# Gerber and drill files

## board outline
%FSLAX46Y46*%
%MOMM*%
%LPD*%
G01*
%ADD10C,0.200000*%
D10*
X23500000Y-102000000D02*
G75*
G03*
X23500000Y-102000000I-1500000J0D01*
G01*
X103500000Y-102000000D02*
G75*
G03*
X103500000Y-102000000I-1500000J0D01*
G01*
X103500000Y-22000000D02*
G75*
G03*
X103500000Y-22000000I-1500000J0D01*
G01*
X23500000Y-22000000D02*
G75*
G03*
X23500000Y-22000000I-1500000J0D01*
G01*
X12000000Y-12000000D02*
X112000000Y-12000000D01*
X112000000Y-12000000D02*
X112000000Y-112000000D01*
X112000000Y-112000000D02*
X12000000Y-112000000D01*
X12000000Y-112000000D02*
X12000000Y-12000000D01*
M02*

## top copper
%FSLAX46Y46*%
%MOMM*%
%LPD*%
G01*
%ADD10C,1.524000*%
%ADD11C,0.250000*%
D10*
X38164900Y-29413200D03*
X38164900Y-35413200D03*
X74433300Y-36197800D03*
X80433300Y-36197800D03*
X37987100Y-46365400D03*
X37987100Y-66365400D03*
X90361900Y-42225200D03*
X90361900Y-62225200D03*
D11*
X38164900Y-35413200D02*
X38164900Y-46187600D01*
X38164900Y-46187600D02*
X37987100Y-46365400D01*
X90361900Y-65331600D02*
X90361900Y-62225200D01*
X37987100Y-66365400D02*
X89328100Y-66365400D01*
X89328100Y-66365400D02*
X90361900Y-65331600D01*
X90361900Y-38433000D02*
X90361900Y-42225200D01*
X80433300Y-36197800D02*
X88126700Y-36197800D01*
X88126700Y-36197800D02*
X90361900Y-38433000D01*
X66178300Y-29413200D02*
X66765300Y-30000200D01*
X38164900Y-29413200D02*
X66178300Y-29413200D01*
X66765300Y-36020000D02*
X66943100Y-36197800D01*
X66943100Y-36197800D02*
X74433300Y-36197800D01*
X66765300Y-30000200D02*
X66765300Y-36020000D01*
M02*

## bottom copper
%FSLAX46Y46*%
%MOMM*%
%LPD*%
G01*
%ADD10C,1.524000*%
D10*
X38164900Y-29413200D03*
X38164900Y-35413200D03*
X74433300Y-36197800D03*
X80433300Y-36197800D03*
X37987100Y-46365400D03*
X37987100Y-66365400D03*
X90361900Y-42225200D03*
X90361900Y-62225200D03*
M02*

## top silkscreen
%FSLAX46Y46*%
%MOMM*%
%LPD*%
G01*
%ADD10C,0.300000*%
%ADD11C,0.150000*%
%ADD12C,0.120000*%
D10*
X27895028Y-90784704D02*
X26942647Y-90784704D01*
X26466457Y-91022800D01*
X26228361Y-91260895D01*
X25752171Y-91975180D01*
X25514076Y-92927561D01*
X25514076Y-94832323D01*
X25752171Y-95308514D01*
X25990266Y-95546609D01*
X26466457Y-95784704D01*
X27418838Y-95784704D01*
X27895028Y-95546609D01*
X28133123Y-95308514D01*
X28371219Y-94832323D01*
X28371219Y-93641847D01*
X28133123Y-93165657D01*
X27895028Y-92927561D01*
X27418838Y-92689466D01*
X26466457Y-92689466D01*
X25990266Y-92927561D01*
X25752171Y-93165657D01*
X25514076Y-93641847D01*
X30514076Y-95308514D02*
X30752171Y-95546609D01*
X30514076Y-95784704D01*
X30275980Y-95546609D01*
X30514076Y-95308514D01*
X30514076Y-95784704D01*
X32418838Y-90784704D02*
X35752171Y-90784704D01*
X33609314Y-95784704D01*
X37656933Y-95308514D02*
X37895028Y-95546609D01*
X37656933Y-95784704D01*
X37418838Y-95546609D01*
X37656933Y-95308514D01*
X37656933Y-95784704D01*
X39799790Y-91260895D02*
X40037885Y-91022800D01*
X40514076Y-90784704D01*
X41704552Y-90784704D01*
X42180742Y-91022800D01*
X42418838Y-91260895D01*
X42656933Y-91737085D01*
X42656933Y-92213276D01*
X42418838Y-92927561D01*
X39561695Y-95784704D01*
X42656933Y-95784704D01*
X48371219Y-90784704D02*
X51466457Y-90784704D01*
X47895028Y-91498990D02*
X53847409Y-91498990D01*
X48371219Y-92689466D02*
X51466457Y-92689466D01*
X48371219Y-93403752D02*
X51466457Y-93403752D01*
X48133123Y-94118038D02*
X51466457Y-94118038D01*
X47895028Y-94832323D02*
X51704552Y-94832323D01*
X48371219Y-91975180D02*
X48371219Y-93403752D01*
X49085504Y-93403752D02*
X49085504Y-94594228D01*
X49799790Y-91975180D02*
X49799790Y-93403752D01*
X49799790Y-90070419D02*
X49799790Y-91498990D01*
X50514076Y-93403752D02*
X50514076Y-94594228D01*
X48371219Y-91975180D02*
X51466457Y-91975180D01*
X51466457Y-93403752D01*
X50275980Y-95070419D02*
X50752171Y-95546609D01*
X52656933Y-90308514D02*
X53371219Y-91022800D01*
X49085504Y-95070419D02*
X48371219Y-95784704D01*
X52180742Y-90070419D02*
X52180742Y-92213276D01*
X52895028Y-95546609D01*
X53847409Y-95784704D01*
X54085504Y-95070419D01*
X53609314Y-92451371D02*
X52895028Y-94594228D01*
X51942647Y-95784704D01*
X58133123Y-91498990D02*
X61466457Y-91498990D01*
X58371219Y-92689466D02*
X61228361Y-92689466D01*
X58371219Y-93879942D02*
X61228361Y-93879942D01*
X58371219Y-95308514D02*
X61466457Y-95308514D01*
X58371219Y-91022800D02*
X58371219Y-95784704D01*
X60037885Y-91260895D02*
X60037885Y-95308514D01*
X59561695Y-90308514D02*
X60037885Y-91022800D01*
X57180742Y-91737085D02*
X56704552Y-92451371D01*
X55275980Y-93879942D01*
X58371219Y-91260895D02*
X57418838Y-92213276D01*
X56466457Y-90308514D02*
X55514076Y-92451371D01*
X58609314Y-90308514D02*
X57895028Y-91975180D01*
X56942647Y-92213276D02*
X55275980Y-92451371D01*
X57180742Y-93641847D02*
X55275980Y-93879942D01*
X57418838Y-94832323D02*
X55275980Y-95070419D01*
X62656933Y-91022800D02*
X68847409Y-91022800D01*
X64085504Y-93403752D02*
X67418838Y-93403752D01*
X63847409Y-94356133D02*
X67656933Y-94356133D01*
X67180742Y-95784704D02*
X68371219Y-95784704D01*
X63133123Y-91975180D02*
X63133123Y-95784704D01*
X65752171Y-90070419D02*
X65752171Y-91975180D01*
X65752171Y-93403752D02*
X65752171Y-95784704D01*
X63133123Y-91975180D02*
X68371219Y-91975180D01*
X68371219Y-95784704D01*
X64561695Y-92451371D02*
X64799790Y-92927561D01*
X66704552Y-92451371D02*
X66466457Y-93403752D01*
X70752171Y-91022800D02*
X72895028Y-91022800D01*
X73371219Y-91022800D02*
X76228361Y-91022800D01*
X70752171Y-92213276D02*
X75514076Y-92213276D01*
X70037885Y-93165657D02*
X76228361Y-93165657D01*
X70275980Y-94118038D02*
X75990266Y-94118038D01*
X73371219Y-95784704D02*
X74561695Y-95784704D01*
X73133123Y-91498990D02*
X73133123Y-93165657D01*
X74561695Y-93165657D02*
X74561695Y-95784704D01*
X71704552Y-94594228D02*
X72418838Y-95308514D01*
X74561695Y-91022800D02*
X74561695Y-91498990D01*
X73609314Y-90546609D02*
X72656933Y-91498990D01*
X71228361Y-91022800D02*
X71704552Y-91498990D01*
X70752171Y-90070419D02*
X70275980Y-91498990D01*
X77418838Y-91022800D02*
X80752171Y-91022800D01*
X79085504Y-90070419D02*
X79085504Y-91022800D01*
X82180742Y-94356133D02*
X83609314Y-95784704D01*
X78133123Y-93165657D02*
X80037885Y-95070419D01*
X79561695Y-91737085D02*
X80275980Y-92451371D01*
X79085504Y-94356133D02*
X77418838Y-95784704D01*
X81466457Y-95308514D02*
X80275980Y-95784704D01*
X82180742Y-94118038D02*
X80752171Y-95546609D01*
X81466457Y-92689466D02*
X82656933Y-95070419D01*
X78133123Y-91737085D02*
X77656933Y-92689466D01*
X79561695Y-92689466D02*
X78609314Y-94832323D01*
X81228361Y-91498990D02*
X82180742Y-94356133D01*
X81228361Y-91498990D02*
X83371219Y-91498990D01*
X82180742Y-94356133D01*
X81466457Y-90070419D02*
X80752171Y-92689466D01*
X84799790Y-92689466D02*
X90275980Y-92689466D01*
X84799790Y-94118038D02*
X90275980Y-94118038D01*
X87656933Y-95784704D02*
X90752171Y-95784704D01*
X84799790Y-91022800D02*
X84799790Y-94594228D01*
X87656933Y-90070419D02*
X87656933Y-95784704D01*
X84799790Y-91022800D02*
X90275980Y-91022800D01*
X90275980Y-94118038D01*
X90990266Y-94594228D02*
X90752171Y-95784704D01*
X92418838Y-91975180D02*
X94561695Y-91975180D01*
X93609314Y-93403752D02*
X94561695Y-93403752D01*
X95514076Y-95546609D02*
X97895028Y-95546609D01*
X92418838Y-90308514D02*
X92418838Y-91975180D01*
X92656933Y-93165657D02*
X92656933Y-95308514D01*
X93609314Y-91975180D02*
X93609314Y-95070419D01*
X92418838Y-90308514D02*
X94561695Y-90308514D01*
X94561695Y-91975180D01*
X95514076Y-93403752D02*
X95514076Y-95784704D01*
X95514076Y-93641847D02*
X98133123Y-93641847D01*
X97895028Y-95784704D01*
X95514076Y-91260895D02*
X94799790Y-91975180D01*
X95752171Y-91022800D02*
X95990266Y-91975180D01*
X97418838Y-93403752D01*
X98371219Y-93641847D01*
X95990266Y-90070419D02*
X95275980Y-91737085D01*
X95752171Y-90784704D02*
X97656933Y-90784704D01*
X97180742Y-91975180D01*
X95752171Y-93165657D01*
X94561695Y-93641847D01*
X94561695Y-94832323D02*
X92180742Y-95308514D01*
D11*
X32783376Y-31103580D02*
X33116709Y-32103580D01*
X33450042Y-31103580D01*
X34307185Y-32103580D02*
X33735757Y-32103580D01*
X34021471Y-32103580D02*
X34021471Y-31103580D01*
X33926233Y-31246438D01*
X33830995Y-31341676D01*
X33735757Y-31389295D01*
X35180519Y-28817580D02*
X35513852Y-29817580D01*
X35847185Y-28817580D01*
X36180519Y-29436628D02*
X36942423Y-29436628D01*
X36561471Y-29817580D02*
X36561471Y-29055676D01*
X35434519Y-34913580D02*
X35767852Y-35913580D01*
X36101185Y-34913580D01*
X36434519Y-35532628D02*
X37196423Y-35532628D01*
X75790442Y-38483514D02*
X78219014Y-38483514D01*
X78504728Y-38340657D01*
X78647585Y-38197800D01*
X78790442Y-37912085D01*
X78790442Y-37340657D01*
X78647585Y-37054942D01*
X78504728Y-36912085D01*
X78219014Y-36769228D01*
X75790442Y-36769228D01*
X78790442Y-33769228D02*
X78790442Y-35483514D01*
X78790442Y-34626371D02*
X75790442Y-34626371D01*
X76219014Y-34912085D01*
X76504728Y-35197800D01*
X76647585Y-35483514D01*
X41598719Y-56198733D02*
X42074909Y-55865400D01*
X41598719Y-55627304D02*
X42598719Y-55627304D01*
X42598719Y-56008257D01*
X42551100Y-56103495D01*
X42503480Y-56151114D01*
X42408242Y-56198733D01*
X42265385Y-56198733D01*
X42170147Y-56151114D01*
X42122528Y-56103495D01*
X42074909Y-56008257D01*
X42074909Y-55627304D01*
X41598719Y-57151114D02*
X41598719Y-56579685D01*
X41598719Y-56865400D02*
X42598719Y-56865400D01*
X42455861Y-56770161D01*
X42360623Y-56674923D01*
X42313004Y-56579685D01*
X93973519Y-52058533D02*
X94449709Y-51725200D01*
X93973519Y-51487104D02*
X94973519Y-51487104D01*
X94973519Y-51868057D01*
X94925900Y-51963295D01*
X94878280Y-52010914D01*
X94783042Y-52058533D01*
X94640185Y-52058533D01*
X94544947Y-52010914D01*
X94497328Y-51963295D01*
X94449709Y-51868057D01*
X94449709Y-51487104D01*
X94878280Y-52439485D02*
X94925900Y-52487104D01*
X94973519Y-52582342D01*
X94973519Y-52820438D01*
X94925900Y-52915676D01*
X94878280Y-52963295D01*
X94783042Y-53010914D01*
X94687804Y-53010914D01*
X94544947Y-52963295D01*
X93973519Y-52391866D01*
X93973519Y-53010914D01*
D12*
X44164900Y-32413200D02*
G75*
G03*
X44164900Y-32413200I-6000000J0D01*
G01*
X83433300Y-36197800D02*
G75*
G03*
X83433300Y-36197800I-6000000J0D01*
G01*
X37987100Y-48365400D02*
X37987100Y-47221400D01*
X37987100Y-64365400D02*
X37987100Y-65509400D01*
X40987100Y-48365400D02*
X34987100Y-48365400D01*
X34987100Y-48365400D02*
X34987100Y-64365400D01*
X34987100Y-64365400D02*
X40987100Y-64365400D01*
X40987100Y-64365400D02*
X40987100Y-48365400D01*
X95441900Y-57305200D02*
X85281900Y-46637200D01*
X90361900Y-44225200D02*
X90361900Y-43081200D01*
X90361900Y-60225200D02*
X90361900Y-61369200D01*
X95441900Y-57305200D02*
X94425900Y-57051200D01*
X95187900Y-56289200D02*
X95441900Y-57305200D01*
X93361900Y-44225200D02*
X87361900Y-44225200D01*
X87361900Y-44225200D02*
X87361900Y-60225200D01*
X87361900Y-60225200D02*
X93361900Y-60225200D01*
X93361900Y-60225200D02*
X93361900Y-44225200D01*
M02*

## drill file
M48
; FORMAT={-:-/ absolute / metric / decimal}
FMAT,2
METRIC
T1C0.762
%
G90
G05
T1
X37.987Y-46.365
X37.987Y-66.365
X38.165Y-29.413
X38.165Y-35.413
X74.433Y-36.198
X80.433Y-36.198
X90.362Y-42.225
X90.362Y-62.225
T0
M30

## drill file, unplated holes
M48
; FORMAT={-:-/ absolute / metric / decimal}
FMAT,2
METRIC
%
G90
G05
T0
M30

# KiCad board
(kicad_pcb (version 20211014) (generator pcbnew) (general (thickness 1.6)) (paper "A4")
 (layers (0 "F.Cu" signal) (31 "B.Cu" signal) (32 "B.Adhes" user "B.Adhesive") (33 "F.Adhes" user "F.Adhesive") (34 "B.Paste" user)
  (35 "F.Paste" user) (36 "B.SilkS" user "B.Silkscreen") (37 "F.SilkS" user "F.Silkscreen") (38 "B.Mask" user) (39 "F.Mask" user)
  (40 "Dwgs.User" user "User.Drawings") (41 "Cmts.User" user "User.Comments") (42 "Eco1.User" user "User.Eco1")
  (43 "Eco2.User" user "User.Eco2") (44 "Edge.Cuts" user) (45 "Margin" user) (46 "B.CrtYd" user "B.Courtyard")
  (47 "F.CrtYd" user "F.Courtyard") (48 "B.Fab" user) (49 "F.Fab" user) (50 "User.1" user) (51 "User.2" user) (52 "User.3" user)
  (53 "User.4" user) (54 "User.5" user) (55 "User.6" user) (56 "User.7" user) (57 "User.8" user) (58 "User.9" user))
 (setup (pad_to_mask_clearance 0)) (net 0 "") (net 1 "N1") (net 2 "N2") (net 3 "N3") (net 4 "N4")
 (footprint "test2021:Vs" (layer "F.Cu") (at 38.1649 32.4132)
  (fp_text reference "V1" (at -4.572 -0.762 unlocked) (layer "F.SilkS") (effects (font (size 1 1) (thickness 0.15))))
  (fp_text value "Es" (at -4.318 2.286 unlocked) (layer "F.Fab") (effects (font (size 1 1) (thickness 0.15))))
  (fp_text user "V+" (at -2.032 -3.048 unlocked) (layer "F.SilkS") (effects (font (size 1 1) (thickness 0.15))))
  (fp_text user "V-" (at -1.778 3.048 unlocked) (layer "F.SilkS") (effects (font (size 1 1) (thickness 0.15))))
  (fp_circle (center 0 0) (end 6 0) (layer "F.SilkS") (width 0.12) (fill none))
  (pad "1" thru_hole circle (at 0 -3) (size 1.524 1.524) (drill 0.762) (layers *.Cu *.Mask) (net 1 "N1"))
  (pad "2" thru_hole circle (at 0 3) (size 1.524 1.524) (drill 0.762) (layers *.Cu *.Mask) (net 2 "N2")))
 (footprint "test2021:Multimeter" (layer "F.Cu") (at 77.4333 36.1978 90)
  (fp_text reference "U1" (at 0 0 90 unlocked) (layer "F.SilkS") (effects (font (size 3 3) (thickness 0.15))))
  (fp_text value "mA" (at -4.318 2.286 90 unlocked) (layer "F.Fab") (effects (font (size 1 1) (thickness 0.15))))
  (fp_circle (center 0 0) (end 6 0) (layer "F.SilkS") (width 0.12) (fill none))
  (pad "1" thru_hole circle (at 0 -3 90) (size 1.524 1.524) (drill 0.762) (layers *.Cu *.Mask) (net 1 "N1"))
  (pad "2" thru_hole circle (at 0 3 90) (size 1.524 1.524) (drill 0.762) (layers *.Cu *.Mask) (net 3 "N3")))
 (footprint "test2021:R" (layer "F.Cu") (at 37.9871 56.3654 -90)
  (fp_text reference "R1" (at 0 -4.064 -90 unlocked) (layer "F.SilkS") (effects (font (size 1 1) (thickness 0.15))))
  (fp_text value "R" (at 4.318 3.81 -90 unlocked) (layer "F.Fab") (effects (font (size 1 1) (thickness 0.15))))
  (fp_line (start -8 0) (end -9.144 0) (layer "F.SilkS") (width 0.12))
  (fp_line (start 8 0) (end 9.144 0) (layer "F.SilkS") (width 0.12))
  (fp_rect (start -8 -3) (end 8 3) (layer "F.SilkS") (width 0.12) (fill none))
  (pad "1" thru_hole circle (at -10 0 270) (size 1.524 1.524) (drill 0.762) (layers *.Cu *.Mask) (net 2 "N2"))
  (pad "2" thru_hole circle (at 10 0 270) (size 1.524 1.524) (drill 0.762) (layers *.Cu *.Mask) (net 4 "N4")))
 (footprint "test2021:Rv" (layer "F.Cu") (at 90.3619 52.2252 -90)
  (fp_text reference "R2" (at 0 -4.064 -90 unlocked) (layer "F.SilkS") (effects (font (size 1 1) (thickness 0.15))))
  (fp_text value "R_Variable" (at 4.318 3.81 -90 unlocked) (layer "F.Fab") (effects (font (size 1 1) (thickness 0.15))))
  (fp_line (start 5.08 -5.08) (end -5.588 5.08) (layer "F.SilkS") (width 0.12))
  (fp_line (start -8 0) (end -9.144 0) (layer "F.SilkS") (width 0.12))
  (fp_line (start 8 0) (end 9.144 0) (layer "F.SilkS") (width 0.12))
  (fp_line (start 5.08 -5.08) (end 4.826 -4.064) (layer "F.SilkS") (width 0.12))
  (fp_line (start 4.064 -4.826) (end 5.08 -5.08) (layer "F.SilkS") (width 0.12))
  (fp_rect (start -8 -3) (end 8 3) (layer "F.SilkS") (width 0.12) (fill none))
  (pad "1" thru_hole circle (at -10 0 270) (size 1.524 1.524) (drill 0.762) (layers *.Cu *.Mask) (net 3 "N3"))
  (pad "2" thru_hole circle (at 10 0 270) (size 1.524 1.524) (drill 0.762) (layers *.Cu *.Mask) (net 4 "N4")))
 (gr_circle (center 22 102) (end 23.5 102) (layer "Edge.Cuts") (width 0.2) (fill none))
 (gr_circle (center 102 102) (end 103.5 102) (layer "Edge.Cuts") (width 0.2) (fill none))
 (gr_circle (center 102 22) (end 103.5 22) (layer "Edge.Cuts") (width 0.2) (fill none))
 (gr_circle (center 22 22) (end 23.5 22) (layer "Edge.Cuts") (width 0.2) (fill none))
 (gr_rect (start 12 12) (end 112 112) (layer "Edge.Cuts") (width 0.2) (fill none))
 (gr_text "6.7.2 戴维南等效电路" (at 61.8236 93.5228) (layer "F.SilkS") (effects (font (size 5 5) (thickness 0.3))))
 (segment (start 38.1649 35.4132) (end 38.1649 46.1876) (width 0.25) (layer "F.Cu") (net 2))
 (segment (start 38.1649 46.1876) (end 37.9871 46.3654) (width 0.25) (layer "F.Cu") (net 2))
 (segment (start 90.3619 65.3316) (end 90.3619 62.2252) (width 0.25) (layer "F.Cu") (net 4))
 (segment (start 37.9871 66.3654) (end 89.3281 66.3654) (width 0.25) (layer "F.Cu") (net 4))
 (segment (start 89.3281 66.3654) (end 90.3619 65.3316) (width 0.25) (layer "F.Cu") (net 4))
 (segment (start 90.3619 38.433) (end 90.3619 42.2252) (width 0.25) (layer "F.Cu") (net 3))
 (segment (start 80.4333 36.1978) (end 88.1267 36.1978) (width 0.25) (layer "F.Cu") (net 3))
 (segment (start 88.1267 36.1978) (end 90.3619 38.433) (width 0.25) (layer "F.Cu") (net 3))
 (segment (start 66.1783 29.4132) (end 66.7653 30.0002) (width 0.25) (layer "F.Cu") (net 1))
 (segment (start 38.1649 29.4132) (end 66.1783 29.4132) (width 0.25) (layer "F.Cu") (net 1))
 (segment (start 66.7653 36.02) (end 66.9431 36.1978) (width 0.25) (layer "F.Cu") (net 1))
 (segment (start 66.9431 36.1978) (end 74.4333 36.1978) (width 0.25) (layer "F.Cu") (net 1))
 (segment (start 66.7653 30.0002) (end 66.7653 36.02) (width 0.25) (layer "F.Cu") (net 1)))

